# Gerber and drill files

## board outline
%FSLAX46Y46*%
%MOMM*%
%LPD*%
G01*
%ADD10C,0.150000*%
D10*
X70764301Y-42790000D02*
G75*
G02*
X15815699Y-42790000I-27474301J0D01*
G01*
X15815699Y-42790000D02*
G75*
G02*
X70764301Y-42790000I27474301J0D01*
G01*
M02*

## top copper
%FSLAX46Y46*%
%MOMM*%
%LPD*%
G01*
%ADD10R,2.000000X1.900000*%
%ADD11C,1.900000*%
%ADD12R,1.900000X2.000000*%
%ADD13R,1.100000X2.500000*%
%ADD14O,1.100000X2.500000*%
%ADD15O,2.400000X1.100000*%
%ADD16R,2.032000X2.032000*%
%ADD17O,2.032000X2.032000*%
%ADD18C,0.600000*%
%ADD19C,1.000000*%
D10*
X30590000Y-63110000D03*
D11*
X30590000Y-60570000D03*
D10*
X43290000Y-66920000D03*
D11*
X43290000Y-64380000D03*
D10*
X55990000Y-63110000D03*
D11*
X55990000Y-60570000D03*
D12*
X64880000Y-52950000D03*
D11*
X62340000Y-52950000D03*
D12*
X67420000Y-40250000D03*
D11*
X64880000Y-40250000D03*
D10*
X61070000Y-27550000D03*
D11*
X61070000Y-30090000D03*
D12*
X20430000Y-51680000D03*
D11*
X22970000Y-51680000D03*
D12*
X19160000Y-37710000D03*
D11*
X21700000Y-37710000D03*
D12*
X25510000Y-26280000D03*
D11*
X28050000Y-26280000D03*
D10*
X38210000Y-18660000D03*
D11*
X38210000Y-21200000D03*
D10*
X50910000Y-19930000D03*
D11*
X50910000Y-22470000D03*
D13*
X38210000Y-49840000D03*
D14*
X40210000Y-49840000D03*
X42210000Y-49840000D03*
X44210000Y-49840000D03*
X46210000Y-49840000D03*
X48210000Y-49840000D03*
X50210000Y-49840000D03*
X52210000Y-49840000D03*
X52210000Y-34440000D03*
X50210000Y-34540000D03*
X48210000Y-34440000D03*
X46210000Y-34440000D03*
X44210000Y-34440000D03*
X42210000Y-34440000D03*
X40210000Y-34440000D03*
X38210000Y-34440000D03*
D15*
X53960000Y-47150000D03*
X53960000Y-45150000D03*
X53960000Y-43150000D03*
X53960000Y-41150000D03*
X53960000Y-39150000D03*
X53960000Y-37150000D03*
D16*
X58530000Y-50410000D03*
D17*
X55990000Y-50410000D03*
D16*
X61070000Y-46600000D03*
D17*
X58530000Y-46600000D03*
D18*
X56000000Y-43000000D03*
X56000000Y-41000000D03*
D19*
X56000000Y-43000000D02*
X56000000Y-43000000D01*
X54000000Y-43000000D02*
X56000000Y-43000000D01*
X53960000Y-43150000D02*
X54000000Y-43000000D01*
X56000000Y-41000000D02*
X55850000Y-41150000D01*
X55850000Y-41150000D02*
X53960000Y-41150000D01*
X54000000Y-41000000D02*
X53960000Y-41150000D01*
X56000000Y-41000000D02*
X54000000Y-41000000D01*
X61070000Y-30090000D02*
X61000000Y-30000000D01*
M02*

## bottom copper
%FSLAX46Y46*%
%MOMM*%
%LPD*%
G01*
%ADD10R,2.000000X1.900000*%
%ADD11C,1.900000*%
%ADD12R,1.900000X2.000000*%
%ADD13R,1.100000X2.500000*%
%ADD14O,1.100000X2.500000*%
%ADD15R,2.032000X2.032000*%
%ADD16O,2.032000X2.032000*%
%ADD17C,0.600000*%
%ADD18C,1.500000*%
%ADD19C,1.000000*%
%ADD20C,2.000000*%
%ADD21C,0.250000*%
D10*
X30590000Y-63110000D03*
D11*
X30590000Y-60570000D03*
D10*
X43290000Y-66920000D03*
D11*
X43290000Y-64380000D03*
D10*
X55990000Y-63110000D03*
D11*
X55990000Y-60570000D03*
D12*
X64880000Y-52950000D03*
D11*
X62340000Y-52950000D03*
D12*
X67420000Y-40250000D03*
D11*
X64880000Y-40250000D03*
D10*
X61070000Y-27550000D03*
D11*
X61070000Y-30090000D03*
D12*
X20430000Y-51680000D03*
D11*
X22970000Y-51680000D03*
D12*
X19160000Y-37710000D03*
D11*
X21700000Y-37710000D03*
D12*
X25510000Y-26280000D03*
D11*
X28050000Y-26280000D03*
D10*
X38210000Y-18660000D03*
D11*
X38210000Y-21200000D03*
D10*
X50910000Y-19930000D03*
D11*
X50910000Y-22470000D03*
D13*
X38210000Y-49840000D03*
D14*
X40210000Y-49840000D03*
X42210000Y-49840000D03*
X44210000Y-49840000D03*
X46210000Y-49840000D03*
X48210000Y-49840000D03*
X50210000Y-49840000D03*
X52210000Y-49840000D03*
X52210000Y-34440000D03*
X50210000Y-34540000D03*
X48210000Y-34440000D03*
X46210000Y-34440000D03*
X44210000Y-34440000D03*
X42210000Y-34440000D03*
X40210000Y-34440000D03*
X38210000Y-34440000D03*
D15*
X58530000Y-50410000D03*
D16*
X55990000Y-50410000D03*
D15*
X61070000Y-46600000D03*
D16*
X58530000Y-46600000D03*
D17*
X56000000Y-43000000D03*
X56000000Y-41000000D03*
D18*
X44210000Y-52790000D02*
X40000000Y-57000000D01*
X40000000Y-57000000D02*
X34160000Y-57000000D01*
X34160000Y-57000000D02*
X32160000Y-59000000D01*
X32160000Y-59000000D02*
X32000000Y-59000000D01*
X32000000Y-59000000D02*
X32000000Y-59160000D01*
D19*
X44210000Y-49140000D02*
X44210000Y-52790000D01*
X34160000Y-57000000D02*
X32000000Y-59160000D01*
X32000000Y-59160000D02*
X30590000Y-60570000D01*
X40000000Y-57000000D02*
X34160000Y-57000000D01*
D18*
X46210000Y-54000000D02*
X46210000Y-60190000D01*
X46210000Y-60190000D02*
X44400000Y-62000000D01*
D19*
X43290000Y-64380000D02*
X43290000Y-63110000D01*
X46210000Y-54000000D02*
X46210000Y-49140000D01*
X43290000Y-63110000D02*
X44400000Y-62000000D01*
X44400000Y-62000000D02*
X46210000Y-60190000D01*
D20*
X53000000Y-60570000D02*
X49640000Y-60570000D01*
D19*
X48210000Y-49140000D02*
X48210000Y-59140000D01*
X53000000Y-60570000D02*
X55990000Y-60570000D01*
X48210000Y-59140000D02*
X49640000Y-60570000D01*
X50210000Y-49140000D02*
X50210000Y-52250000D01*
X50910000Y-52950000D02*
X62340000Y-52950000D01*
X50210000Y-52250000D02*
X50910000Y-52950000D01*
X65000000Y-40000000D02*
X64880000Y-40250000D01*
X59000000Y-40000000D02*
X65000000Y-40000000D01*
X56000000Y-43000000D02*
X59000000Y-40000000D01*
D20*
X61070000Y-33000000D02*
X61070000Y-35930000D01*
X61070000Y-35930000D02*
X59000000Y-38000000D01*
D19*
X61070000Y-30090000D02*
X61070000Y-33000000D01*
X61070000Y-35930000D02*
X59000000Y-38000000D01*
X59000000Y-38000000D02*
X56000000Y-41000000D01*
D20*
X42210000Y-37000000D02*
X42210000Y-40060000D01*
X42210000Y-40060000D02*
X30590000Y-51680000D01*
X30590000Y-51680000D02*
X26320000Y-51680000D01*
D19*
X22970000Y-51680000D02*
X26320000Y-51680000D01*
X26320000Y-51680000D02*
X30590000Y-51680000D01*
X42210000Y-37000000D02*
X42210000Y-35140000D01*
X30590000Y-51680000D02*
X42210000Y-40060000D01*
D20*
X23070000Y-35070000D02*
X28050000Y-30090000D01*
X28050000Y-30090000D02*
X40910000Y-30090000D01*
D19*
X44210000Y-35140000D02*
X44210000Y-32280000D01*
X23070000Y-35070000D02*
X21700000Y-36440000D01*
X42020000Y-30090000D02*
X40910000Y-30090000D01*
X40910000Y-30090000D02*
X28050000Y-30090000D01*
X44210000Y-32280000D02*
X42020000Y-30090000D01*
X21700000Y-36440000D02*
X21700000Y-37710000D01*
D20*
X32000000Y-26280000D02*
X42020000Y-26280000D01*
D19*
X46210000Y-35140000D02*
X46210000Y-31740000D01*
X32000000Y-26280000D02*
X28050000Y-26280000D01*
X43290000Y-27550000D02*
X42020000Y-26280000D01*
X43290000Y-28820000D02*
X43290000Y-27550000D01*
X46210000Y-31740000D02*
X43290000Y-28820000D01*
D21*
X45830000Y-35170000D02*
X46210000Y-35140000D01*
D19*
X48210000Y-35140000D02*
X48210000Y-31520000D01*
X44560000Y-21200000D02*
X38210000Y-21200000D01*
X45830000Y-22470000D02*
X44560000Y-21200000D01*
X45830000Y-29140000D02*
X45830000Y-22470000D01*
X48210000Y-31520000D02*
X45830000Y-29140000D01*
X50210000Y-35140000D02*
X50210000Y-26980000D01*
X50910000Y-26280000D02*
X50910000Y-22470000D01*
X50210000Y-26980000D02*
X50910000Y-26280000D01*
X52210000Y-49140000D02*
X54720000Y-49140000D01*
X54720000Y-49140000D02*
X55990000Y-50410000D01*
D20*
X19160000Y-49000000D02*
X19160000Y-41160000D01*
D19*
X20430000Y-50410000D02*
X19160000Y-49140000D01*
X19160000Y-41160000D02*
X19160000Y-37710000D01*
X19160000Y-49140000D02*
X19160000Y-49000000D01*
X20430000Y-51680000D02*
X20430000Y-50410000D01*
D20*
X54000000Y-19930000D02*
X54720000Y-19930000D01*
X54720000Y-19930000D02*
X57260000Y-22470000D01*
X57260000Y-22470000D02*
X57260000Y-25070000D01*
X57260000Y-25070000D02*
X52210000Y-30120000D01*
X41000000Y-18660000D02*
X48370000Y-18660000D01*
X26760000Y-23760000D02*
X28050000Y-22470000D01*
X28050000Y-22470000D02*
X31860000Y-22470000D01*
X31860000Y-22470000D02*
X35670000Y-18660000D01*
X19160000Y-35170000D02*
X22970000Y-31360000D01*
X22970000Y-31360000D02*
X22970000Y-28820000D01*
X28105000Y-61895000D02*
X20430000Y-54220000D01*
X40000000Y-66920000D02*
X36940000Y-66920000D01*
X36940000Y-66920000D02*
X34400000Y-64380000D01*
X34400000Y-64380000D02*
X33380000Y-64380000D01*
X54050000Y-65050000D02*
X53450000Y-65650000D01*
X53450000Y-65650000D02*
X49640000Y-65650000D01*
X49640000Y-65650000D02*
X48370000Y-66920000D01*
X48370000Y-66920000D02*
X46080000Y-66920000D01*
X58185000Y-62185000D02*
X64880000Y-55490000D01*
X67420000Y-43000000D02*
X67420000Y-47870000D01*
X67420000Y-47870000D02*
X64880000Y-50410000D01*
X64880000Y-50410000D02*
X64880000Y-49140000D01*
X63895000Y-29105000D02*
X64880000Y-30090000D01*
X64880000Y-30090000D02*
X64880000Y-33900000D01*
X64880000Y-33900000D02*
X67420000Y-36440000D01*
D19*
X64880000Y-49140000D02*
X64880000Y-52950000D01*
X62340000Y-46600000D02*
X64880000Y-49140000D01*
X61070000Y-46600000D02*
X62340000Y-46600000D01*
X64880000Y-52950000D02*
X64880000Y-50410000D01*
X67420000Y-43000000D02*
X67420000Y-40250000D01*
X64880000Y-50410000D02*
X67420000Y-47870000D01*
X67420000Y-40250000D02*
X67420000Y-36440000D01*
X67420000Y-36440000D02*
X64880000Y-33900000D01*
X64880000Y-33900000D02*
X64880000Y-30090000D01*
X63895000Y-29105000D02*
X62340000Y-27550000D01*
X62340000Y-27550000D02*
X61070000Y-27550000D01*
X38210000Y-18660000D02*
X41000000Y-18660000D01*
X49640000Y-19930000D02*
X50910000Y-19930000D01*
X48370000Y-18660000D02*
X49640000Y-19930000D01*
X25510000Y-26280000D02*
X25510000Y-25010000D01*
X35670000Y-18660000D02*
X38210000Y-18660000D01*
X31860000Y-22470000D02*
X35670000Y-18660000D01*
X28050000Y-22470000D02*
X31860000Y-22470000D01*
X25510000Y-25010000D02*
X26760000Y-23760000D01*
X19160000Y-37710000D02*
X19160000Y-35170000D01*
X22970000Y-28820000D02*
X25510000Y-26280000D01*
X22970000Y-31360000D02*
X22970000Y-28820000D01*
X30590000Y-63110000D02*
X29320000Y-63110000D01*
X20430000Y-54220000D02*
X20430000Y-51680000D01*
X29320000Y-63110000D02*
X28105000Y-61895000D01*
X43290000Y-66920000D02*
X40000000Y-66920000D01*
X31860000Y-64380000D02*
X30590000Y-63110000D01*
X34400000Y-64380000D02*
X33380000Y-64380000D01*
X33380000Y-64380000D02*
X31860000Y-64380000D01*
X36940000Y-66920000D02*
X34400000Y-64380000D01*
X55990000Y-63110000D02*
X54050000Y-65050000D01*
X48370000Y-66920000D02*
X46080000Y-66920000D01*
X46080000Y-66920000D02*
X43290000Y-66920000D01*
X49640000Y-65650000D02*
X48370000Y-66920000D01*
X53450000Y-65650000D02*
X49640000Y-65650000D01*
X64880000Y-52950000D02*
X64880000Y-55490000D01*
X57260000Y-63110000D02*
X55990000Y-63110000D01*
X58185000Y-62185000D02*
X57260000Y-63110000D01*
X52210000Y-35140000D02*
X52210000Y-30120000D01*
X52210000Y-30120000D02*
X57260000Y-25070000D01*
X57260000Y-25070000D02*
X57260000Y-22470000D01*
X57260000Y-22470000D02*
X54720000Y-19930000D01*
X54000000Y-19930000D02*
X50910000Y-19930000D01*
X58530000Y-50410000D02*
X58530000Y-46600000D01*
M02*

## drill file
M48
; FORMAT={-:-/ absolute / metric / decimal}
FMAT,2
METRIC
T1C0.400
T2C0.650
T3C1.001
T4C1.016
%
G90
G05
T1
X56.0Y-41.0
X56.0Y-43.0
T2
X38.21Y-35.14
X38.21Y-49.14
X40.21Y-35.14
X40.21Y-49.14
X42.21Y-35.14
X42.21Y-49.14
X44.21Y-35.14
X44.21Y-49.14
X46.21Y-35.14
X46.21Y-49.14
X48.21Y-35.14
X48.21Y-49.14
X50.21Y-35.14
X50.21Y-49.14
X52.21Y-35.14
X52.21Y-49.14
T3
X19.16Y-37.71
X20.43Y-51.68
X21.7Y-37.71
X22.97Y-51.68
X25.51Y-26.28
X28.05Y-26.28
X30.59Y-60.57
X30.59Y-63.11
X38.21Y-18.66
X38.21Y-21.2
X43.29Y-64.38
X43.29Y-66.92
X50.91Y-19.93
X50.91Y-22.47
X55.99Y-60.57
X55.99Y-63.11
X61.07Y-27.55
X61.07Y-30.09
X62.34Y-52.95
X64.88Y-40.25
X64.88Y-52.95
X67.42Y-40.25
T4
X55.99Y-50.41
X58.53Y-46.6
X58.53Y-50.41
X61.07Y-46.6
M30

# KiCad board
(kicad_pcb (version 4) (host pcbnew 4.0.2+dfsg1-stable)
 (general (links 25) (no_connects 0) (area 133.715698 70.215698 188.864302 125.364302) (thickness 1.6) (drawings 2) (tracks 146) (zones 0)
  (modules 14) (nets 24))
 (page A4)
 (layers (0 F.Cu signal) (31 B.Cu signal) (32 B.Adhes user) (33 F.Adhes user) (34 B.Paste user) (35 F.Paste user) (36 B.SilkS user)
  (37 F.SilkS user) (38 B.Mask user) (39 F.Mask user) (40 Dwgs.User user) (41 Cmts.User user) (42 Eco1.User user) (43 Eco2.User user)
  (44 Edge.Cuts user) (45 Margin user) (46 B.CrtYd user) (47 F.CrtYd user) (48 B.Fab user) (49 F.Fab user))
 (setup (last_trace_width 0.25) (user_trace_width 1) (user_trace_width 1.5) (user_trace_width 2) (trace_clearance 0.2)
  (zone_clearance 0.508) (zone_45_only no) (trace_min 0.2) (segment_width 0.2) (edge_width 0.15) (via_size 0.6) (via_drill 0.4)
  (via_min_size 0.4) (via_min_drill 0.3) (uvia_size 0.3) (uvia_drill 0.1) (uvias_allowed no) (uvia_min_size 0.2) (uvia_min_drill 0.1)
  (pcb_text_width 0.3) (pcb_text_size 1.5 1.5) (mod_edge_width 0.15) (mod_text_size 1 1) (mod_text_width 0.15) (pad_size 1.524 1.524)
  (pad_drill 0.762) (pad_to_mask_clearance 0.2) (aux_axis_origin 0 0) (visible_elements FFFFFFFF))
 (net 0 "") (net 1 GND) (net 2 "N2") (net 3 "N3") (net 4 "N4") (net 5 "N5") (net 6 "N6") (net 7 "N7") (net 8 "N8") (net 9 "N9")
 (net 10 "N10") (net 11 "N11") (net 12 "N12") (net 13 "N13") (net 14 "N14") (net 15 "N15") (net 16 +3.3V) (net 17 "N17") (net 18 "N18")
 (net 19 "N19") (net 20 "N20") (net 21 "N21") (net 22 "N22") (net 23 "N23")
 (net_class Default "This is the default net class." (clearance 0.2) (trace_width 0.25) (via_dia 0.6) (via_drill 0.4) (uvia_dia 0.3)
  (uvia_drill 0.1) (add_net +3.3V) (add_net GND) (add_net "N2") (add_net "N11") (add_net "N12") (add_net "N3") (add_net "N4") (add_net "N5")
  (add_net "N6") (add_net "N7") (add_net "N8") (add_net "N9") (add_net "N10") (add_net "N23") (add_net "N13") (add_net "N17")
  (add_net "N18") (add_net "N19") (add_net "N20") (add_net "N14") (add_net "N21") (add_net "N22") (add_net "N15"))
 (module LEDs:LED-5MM (layer F.Cu) (at 30.59 63.11 90)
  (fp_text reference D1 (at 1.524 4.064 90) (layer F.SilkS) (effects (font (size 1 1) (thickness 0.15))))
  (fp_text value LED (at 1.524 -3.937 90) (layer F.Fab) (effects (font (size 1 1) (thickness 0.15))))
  (pad 1 thru_hole rect (at 0 0 180) (size 2 1.9) (drill 1.00076) (layers *.Cu *.Mask F.SilkS) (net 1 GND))
  (pad 2 thru_hole circle (at 2.54 0 90) (size 1.9 1.9) (drill 1.00076) (layers *.Cu *.Mask F.SilkS) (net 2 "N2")))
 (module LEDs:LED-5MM (layer F.Cu) (at 43.29 66.92 90)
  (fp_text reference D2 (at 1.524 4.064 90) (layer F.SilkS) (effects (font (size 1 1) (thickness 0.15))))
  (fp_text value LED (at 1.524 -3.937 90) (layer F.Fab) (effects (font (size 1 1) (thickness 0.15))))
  (pad 1 thru_hole rect (at 0 0 180) (size 2 1.9) (drill 1.00076) (layers *.Cu *.Mask F.SilkS) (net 1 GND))
  (pad 2 thru_hole circle (at 2.54 0 90) (size 1.9 1.9) (drill 1.00076) (layers *.Cu *.Mask F.SilkS) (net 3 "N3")))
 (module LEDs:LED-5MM (layer F.Cu) (at 55.99 63.11 90)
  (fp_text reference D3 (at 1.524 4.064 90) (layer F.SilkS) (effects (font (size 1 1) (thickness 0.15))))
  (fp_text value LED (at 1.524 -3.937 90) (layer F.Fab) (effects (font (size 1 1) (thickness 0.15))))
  (pad 1 thru_hole rect (at 0 0 180) (size 2 1.9) (drill 1.00076) (layers *.Cu *.Mask F.SilkS) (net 1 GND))
  (pad 2 thru_hole circle (at 2.54 0 90) (size 1.9 1.9) (drill 1.00076) (layers *.Cu *.Mask F.SilkS) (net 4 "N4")))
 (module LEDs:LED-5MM (layer F.Cu) (at 64.88 52.95 180)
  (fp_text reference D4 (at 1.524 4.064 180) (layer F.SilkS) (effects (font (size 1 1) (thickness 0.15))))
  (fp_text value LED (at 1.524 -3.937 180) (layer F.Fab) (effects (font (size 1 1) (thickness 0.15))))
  (pad 1 thru_hole rect (at 0 0 270) (size 2 1.9) (drill 1.00076) (layers *.Cu *.Mask F.SilkS) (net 1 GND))
  (pad 2 thru_hole circle (at 2.54 0 180) (size 1.9 1.9) (drill 1.00076) (layers *.Cu *.Mask F.SilkS) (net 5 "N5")))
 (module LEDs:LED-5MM (layer F.Cu) (at 67.42 40.25 180)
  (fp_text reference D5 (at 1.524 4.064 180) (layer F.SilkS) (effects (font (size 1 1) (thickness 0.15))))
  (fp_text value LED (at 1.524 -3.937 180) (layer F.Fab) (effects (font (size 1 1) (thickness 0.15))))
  (pad 1 thru_hole rect (at 0 0 270) (size 2 1.9) (drill 1.00076) (layers *.Cu *.Mask F.SilkS) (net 1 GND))
  (pad 2 thru_hole circle (at 2.54 0 180) (size 1.9 1.9) (drill 1.00076) (layers *.Cu *.Mask F.SilkS) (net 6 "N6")))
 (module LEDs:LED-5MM (layer F.Cu) (at 61.07 27.55 270)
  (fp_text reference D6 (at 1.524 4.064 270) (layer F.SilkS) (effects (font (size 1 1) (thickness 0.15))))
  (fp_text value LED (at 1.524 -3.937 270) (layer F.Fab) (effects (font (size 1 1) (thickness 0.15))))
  (pad 1 thru_hole rect (at 0 0) (size 2 1.9) (drill 1.00076) (layers *.Cu *.Mask F.SilkS) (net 1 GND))
  (pad 2 thru_hole circle (at 2.54 0 270) (size 1.9 1.9) (drill 1.00076) (layers *.Cu *.Mask F.SilkS) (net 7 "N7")))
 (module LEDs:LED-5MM (layer F.Cu) (at 20.43 51.68)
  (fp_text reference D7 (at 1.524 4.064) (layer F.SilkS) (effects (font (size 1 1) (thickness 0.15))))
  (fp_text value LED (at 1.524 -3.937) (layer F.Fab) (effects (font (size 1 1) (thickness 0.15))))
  (pad 1 thru_hole rect (at 0 0 90) (size 2 1.9) (drill 1.00076) (layers *.Cu *.Mask F.SilkS) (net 1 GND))
  (pad 2 thru_hole circle (at 2.54 0) (size 1.9 1.9) (drill 1.00076) (layers *.Cu *.Mask F.SilkS) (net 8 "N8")))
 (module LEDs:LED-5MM (layer F.Cu) (at 19.16 37.71)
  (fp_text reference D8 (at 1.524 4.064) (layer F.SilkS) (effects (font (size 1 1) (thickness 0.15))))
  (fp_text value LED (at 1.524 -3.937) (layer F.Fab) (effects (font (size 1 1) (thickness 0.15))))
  (pad 1 thru_hole rect (at 0 0 90) (size 2 1.9) (drill 1.00076) (layers *.Cu *.Mask F.SilkS) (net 1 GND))
  (pad 2 thru_hole circle (at 2.54 0) (size 1.9 1.9) (drill 1.00076) (layers *.Cu *.Mask F.SilkS) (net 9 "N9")))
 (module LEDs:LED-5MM (layer F.Cu) (at 25.51 26.28)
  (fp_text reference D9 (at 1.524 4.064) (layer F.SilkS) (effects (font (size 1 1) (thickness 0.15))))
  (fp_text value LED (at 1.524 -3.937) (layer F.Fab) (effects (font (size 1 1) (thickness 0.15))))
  (pad 1 thru_hole rect (at 0 0 90) (size 2 1.9) (drill 1.00076) (layers *.Cu *.Mask F.SilkS) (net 1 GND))
  (pad 2 thru_hole circle (at 2.54 0) (size 1.9 1.9) (drill 1.00076) (layers *.Cu *.Mask F.SilkS) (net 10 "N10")))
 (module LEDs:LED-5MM (layer F.Cu) (at 38.21 18.66 270)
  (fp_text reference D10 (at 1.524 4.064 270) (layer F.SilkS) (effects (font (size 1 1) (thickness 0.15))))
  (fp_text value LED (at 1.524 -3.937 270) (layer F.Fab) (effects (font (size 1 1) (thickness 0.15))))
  (pad 1 thru_hole rect (at 0 0) (size 2 1.9) (drill 1.00076) (layers *.Cu *.Mask F.SilkS) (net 1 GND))
  (pad 2 thru_hole circle (at 2.54 0 270) (size 1.9 1.9) (drill 1.00076) (layers *.Cu *.Mask F.SilkS) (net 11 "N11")))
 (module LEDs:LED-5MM (layer F.Cu) (at 50.91 19.93 270)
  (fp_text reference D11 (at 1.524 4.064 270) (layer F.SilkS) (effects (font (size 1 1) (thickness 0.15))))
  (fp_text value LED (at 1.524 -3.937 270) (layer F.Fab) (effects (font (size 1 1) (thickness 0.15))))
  (pad 1 thru_hole rect (at 0 0) (size 2 1.9) (drill 1.00076) (layers *.Cu *.Mask F.SilkS) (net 1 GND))
  (pad 2 thru_hole circle (at 2.54 0 270) (size 1.9 1.9) (drill 1.00076) (layers *.Cu *.Mask F.SilkS) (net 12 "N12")))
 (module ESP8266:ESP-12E (layer F.Cu) (at 38.21 49.14 90)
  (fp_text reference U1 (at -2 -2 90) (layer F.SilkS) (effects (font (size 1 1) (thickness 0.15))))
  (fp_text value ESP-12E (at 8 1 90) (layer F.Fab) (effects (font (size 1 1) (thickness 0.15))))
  (pad 1 thru_hole rect (at 0 0 90) (size 2.5 1.1) (drill 0.65 (offset -0.7 0)) (layers *.Cu *.Mask F.SilkS) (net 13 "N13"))
  (pad 2 thru_hole oval (at 0 2 90) (size 2.5 1.1) (drill 0.65 (offset -0.7 0)) (layers *.Cu *.Mask F.SilkS) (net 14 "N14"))
  (pad 3 thru_hole oval (at 0 4 90) (size 2.5 1.1) (drill 0.65 (offset -0.7 0)) (layers *.Cu *.Mask F.SilkS) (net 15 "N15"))
  (pad 4 thru_hole oval (at 0 6 90) (size 2.5 1.1) (drill 0.65 (offset -0.7 0)) (layers *.Cu *.Mask F.SilkS) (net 2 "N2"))
  (pad 5 thru_hole oval (at 0 8 90) (size 2.5 1.1) (drill 0.65 (offset -0.7 0)) (layers *.Cu *.Mask F.SilkS) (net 3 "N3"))
  (pad 6 thru_hole oval (at 0 10 90) (size 2.5 1.1) (drill 0.65 (offset -0.7 0)) (layers *.Cu *.Mask F.SilkS) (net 4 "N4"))
  (pad 7 thru_hole oval (at 0 12 90) (size 2.5 1.1) (drill 0.65 (offset -0.7 0)) (layers *.Cu *.Mask F.SilkS) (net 5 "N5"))
  (pad 8 thru_hole oval (at 0 14 90) (size 2.5 1.1) (drill 0.65 (offset -0.7 0)) (layers *.Cu *.Mask F.SilkS) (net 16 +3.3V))
  (pad 9 thru_hole oval (at 14 14 90) (size 2.5 1.1) (drill 0.65 (offset 0.7 0)) (layers *.Cu *.Mask F.SilkS) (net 1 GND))
  (pad 10 thru_hole oval (at 14 12 90) (size 2.5 1.1) (drill 0.65 (offset 0.6 0)) (layers *.Cu *.Mask F.SilkS) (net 12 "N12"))
  (pad 11 thru_hole oval (at 14 10 90) (size 2.5 1.1) (drill 0.65 (offset 0.7 0)) (layers *.Cu *.Mask F.SilkS) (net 11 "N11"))
  (pad 12 thru_hole oval (at 14 8 90) (size 2.5 1.1) (drill 0.65 (offset 0.7 0)) (layers *.Cu *.Mask F.SilkS) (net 10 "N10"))
  (pad 13 thru_hole oval (at 14 6 90) (size 2.5 1.1) (drill 0.65 (offset 0.7 0)) (layers *.Cu *.Mask F.SilkS) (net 9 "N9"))
  (pad 14 thru_hole oval (at 14 4 90) (size 2.5 1.1) (drill 0.65 (offset 0.7 0)) (layers *.Cu *.Mask F.SilkS) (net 8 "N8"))
  (pad 15 thru_hole oval (at 14 2 90) (size 2.5 1.1) (drill 0.65 (offset 0.7 0)) (layers *.Cu *.Mask F.SilkS) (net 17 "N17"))
  (pad 16 thru_hole oval (at 14 0 90) (size 2.5 1.1) (drill 0.65 (offset 0.7 0)) (layers *.Cu *.Mask F.SilkS) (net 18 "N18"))
  (pad 17 smd oval (at 1.99 15.75 180) (size 2.4 1.1) (layers F.Cu F.Paste F.Mask) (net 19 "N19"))
  (pad 18 smd oval (at 3.99 15.75 180) (size 2.4 1.1) (layers F.Cu F.Paste F.Mask) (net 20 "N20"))
  (pad 19 smd oval (at 5.99 15.75 180) (size 2.4 1.1) (layers F.Cu F.Paste F.Mask) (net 6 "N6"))
  (pad 20 smd oval (at 7.99 15.75 180) (size 2.4 1.1) (layers F.Cu F.Paste F.Mask) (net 7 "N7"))
  (pad 21 smd oval (at 9.99 15.75 180) (size 2.4 1.1) (layers F.Cu F.Paste F.Mask) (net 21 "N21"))
  (pad 22 smd oval (at 11.99 15.75 180) (size 2.4 1.1) (layers F.Cu F.Paste F.Mask) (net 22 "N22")))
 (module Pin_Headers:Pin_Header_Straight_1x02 (layer F.Cu) (at 58.53 50.41 270)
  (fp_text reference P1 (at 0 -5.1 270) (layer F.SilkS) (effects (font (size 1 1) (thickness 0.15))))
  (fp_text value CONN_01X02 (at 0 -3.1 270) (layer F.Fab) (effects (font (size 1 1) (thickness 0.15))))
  (pad 1 thru_hole rect (at 0 0 270) (size 2.032 2.032) (drill 1.016) (layers *.Cu *.Mask F.SilkS) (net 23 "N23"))
  (pad 2 thru_hole oval (at 0 2.54 270) (size 2.032 2.032) (drill 1.016) (layers *.Cu *.Mask F.SilkS) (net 16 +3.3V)))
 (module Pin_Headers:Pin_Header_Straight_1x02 (layer F.Cu) (at 61.07 46.6 270)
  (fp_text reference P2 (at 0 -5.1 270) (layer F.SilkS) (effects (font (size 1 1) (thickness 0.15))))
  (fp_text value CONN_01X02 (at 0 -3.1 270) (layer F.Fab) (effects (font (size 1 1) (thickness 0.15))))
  (pad 1 thru_hole rect (at 0 0 270) (size 2.032 2.032) (drill 1.016) (layers *.Cu *.Mask F.SilkS) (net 1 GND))
  (pad 2 thru_hole oval (at 0 2.54 270) (size 2.032 2.032) (drill 1.016) (layers *.Cu *.Mask F.SilkS) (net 23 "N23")))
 (gr_circle (center 43.29 42.79) (end 66.15 58.03) (layer Edge.Cuts) (width 0.15))
 (segment (start 44.21 52.79) (end 40 57) (width 1.5) (layer B.Cu) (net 2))
 (segment (start 40 57) (end 34.16 57) (width 1.5) (layer B.Cu) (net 2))
 (segment (start 34.16 57) (end 32.16 59) (width 1.5) (layer B.Cu) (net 2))
 (segment (start 32.16 59) (end 32 59) (width 1.5) (layer B.Cu) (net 2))
 (segment (start 32 59) (end 32 59.16) (width 1.5) (layer B.Cu) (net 2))
 (segment (start 44.21 49.14) (end 44.21 52.79) (width 1) (layer B.Cu) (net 2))
 (segment (start 34.16 57) (end 32 59.16) (width 1) (layer B.Cu) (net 2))
 (segment (start 32 59.16) (end 30.59 60.57) (width 1) (layer B.Cu) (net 2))
 (segment (start 40 57) (end 34.16 57) (width 1) (layer B.Cu) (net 2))
 (segment (start 46.21 54) (end 46.21 60.19) (width 1.5) (layer B.Cu) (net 3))
 (segment (start 46.21 60.19) (end 44.4 62) (width 1.5) (layer B.Cu) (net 3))
 (segment (start 43.29 64.38) (end 43.29 63.11) (width 1) (layer B.Cu) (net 3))
 (segment (start 46.21 54) (end 46.21 49.14) (width 1) (layer B.Cu) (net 3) (status 20))
 (segment (start 43.29 63.11) (end 44.4 62) (width 1) (layer B.Cu) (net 3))
 (segment (start 44.4 62) (end 46.21 60.19) (width 1) (layer B.Cu) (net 3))
 (segment (start 53 60.57) (end 49.64 60.57) (width 2) (layer B.Cu) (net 4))
 (segment (start 48.21 49.14) (end 48.21 59.14) (width 1) (layer B.Cu) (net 4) (status 10))
 (segment (start 53 60.57) (end 55.99 60.57) (width 1) (layer B.Cu) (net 4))
 (segment (start 48.21 59.14) (end 49.64 60.57) (width 1) (layer B.Cu) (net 4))
 (segment (start 50.21 49.14) (end 50.21 52.25) (width 1) (layer B.Cu) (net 5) (status 10))
 (segment (start 50.91 52.95) (end 62.34 52.95) (width 1) (layer B.Cu) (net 5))
 (segment (start 50.21 52.25) (end 50.91 52.95) (width 1) (layer B.Cu) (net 5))
 (segment (start 65 40) (end 64.88 40.25) (width 1) (layer B.Cu) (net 6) (status 80000))
 (segment (start 59 40) (end 65 40) (width 1) (layer B.Cu) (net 6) (status 80000))
 (segment (start 56 43) (end 59 40) (width 1) (layer B.Cu) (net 6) (status 80000))
 (via (at 56 43) (size 0.6) (layers F.Cu B.Cu) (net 6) (status 80000))
 (segment (start 56 43) (end 56 43) (width 1) (layer F.Cu) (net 6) (status 80000))
 (segment (start 54 43) (end 56 43) (width 1) (layer F.Cu) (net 6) (status 80000))
 (segment (start 53.96 43.15) (end 54 43) (width 1) (layer F.Cu) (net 6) (status 80000))
 (segment (start 61.07 33) (end 61.07 35.93) (width 2) (layer B.Cu) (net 7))
 (segment (start 61.07 35.93) (end 59 38) (width 2) (layer B.Cu) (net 7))
 (segment (start 61.07 30.09) (end 61.07 33) (width 1) (layer B.Cu) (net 7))
 (via (at 56 41) (size 0.6) (drill 0.4) (layers F.Cu B.Cu) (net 7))
 (segment (start 61.07 35.93) (end 59 38) (width 1) (layer B.Cu) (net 7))
 (segment (start 59 38) (end 56 41) (width 1) (layer B.Cu) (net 7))
 (segment (start 56 41) (end 55.85 41.15) (width 1) (layer F.Cu) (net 7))
 (segment (start 55.85 41.15) (end 53.96 41.15) (width 1) (layer F.Cu) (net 7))
 (segment (start 54 41) (end 53.96 41.15) (width 1) (layer F.Cu) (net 7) (status 80000))
 (segment (start 56 41) (end 54 41) (width 1) (layer F.Cu) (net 7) (status 80000))
 (segment (start 61.07 30.09) (end 61 30) (width 1) (layer F.Cu) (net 7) (status 80000))
 (segment (start 42.21 37) (end 42.21 40.06) (width 2) (layer B.Cu) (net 8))
 (segment (start 42.21 40.06) (end 30.59 51.68) (width 2) (layer B.Cu) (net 8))
 (segment (start 30.59 51.68) (end 26.32 51.68) (width 2) (layer B.Cu) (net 8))
 (segment (start 22.97 51.68) (end 26.32 51.68) (width 1) (layer B.Cu) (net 8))
 (segment (start 26.32 51.68) (end 30.59 51.68) (width 1) (layer B.Cu) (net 8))
 (segment (start 42.21 37) (end 42.21 35.14) (width 1) (layer B.Cu) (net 8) (status 20))
 (segment (start 30.59 51.68) (end 42.21 40.06) (width 1) (layer B.Cu) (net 8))
 (segment (start 23.07 35.07) (end 28.05 30.09) (width 2) (layer B.Cu) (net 9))
 (segment (start 28.05 30.09) (end 40.91 30.09) (width 2) (layer B.Cu) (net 9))
 (segment (start 44.21 35.14) (end 44.21 32.28) (width 1) (layer B.Cu) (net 9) (status 10))
 (segment (start 23.07 35.07) (end 21.7 36.44) (width 1) (layer B.Cu) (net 9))
 (segment (start 42.02 30.09) (end 40.91 30.09) (width 1) (layer B.Cu) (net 9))
 (segment (start 40.91 30.09) (end 28.05 30.09) (width 1) (layer B.Cu) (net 9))
 (segment (start 44.21 32.28) (end 42.02 30.09) (width 1) (layer B.Cu) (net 9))
 (segment (start 21.7 36.44) (end 21.7 37.71) (width 1) (layer B.Cu) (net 9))
 (segment (start 32 26.28) (end 42.02 26.28) (width 2) (layer B.Cu) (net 10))
 (segment (start 46.21 35.14) (end 46.21 31.74) (width 1) (layer B.Cu) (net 10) (status 10))
 (segment (start 32 26.28) (end 28.05 26.28) (width 1) (layer B.Cu) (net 10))
 (segment (start 43.29 27.55) (end 42.02 26.28) (width 1) (layer B.Cu) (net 10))
 (segment (start 43.29 28.82) (end 43.29 27.55) (width 1) (layer B.Cu) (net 10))
 (segment (start 46.21 31.74) (end 43.29 28.82) (width 1) (layer B.Cu) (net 10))
 (segment (start 45.83 35.17) (end 46.21 35.14) (width 0.25) (layer B.Cu) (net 10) (status 80030))
 (segment (start 48.21 35.14) (end 48.21 31.52) (width 1) (layer B.Cu) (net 11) (status 10))
 (segment (start 44.56 21.2) (end 38.21 21.2) (width 1) (layer B.Cu) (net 11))
 (segment (start 45.83 22.47) (end 44.56 21.2) (width 1) (layer B.Cu) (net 11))
 (segment (start 45.83 29.14) (end 45.83 22.47) (width 1) (layer B.Cu) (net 11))
 (segment (start 48.21 31.52) (end 45.83 29.14) (width 1) (layer B.Cu) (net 11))
 (segment (start 50.21 35.14) (end 50.21 26.98) (width 1) (layer B.Cu) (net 12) (status 10))
 (segment (start 50.91 26.28) (end 50.91 22.47) (width 1) (layer B.Cu) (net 12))
 (segment (start 50.21 26.98) (end 50.91 26.28) (width 1) (layer B.Cu) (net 12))
 (segment (start 52.21 49.14) (end 54.72 49.14) (width 1) (layer B.Cu) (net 16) (status 10))
 (segment (start 54.72 49.14) (end 55.99 50.41) (width 1) (layer B.Cu) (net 16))
 (segment (start 19.16 49) (end 19.16 41.16) (width 2) (layer B.Cu) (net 1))
 (segment (start 20.43 50.41) (end 19.16 49.14) (width 1) (layer B.Cu) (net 1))
 (segment (start 19.16 41.16) (end 19.16 37.71) (width 1) (layer B.Cu) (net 1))
 (segment (start 19.16 49.14) (end 19.16 49) (width 1) (layer B.Cu) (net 1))
 (segment (start 20.43 51.68) (end 20.43 50.41) (width 1) (layer B.Cu) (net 1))
 (segment (start 54 19.93) (end 54.72 19.93) (width 2) (layer B.Cu) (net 1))
 (segment (start 54.72 19.93) (end 57.26 22.47) (width 2) (layer B.Cu) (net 1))
 (segment (start 57.26 22.47) (end 57.26 25.07) (width 2) (layer B.Cu) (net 1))
 (segment (start 57.26 25.07) (end 52.21 30.12) (width 2) (layer B.Cu) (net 1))
 (segment (start 41 18.66) (end 48.37 18.66) (width 2) (layer B.Cu) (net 1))
 (segment (start 26.76 23.76) (end 28.05 22.47) (width 2) (layer B.Cu) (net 1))
 (segment (start 28.05 22.47) (end 31.86 22.47) (width 2) (layer B.Cu) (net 1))
 (segment (start 31.86 22.47) (end 35.67 18.66) (width 2) (layer B.Cu) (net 1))
 (segment (start 19.16 35.17) (end 22.97 31.36) (width 2) (layer B.Cu) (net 1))
 (segment (start 22.97 31.36) (end 22.97 28.82) (width 2) (layer B.Cu) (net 1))
 (segment (start 28.105 61.895) (end 20.43 54.22) (width 2) (layer B.Cu) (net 1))
 (segment (start 40 66.92) (end 36.94 66.92) (width 2) (layer B.Cu) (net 1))
 (segment (start 36.94 66.92) (end 34.4 64.38) (width 2) (layer B.Cu) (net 1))
 (segment (start 34.4 64.38) (end 33.38 64.38) (width 2) (layer B.Cu) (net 1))
 (segment (start 54.05 65.05) (end 53.45 65.65) (width 2) (layer B.Cu) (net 1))
 (segment (start 53.45 65.65) (end 49.64 65.65) (width 2) (layer B.Cu) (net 1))
 (segment (start 49.64 65.65) (end 48.37 66.92) (width 2) (layer B.Cu) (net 1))
 (segment (start 48.37 66.92) (end 46.08 66.92) (width 2) (layer B.Cu) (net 1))
 (segment (start 58.185 62.185) (end 64.88 55.49) (width 2) (layer B.Cu) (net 1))
 (segment (start 67.42 43) (end 67.42 47.87) (width 2) (layer B.Cu) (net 1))
 (segment (start 67.42 47.87) (end 64.88 50.41) (width 2) (layer B.Cu) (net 1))
 (segment (start 64.88 50.41) (end 64.88 49.14) (width 2) (layer B.Cu) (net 1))
 (segment (start 63.895 29.105) (end 64.88 30.09) (width 2) (layer B.Cu) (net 1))
 (segment (start 64.88 30.09) (end 64.88 33.9) (width 2) (layer B.Cu) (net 1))
 (segment (start 64.88 33.9) (end 67.42 36.44) (width 2) (layer B.Cu) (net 1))
 (segment (start 64.88 49.14) (end 64.88 52.95) (width 1) (layer B.Cu) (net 1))
 (segment (start 62.34 46.6) (end 64.88 49.14) (width 1) (layer B.Cu) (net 1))
 (segment (start 61.07 46.6) (end 62.34 46.6) (width 1) (layer B.Cu) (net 1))
 (segment (start 64.88 52.95) (end 64.88 50.41) (width 1) (layer B.Cu) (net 1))
 (segment (start 67.42 43) (end 67.42 40.25) (width 1) (layer B.Cu) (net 1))
 (segment (start 64.88 50.41) (end 67.42 47.87) (width 1) (layer B.Cu) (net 1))
 (segment (start 67.42 40.25) (end 67.42 36.44) (width 1) (layer B.Cu) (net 1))
 (segment (start 67.42 36.44) (end 64.88 33.9) (width 1) (layer B.Cu) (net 1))
 (segment (start 64.88 33.9) (end 64.88 30.09) (width 1) (layer B.Cu) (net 1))
 (segment (start 63.895 29.105) (end 62.34 27.55) (width 1) (layer B.Cu) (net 1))
 (segment (start 62.34 27.55) (end 61.07 27.55) (width 1) (layer B.Cu) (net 1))
 (segment (start 38.21 18.66) (end 41 18.66) (width 1) (layer B.Cu) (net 1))
 (segment (start 49.64 19.93) (end 50.91 19.93) (width 1) (layer B.Cu) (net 1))
 (segment (start 48.37 18.66) (end 49.64 19.93) (width 1) (layer B.Cu) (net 1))
 (segment (start 25.51 26.28) (end 25.51 25.01) (width 1) (layer B.Cu) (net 1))
 (segment (start 35.67 18.66) (end 38.21 18.66) (width 1) (layer B.Cu) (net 1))
 (segment (start 31.86 22.47) (end 35.67 18.66) (width 1) (layer B.Cu) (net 1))
 (segment (start 28.05 22.47) (end 31.86 22.47) (width 1) (layer B.Cu) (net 1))
 (segment (start 25.51 25.01) (end 26.76 23.76) (width 1) (layer B.Cu) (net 1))
 (segment (start 19.16 37.71) (end 19.16 35.17) (width 1) (layer B.Cu) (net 1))
 (segment (start 22.97 28.82) (end 25.51 26.28) (width 1) (layer B.Cu) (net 1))
 (segment (start 22.97 31.36) (end 22.97 28.82) (width 1) (layer B.Cu) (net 1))
 (segment (start 30.59 63.11) (end 29.32 63.11) (width 1) (layer B.Cu) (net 1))
 (segment (start 20.43 54.22) (end 20.43 51.68) (width 1) (layer B.Cu) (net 1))
 (segment (start 29.32 63.11) (end 28.105 61.895) (width 1) (layer B.Cu) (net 1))
 (segment (start 43.29 66.92) (end 40 66.92) (width 1) (layer B.Cu) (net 1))
 (segment (start 31.86 64.38) (end 30.59 63.11) (width 1) (layer B.Cu) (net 1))
 (segment (start 34.4 64.38) (end 33.38 64.38) (width 1) (layer B.Cu) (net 1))
 (segment (start 33.38 64.38) (end 31.86 64.38) (width 1) (layer B.Cu) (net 1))
 (segment (start 36.94 66.92) (end 34.4 64.38) (width 1) (layer B.Cu) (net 1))
 (segment (start 55.99 63.11) (end 54.05 65.05) (width 1) (layer B.Cu) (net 1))
 (segment (start 48.37 66.92) (end 46.08 66.92) (width 1) (layer B.Cu) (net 1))
 (segment (start 46.08 66.92) (end 43.29 66.92) (width 1) (layer B.Cu) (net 1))
 (segment (start 49.64 65.65) (end 48.37 66.92) (width 1) (layer B.Cu) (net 1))
 (segment (start 53.45 65.65) (end 49.64 65.65) (width 1) (layer B.Cu) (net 1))
 (segment (start 64.88 52.95) (end 64.88 55.49) (width 1) (layer B.Cu) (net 1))
 (segment (start 57.26 63.11) (end 55.99 63.11) (width 1) (layer B.Cu) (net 1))
 (segment (start 58.185 62.185) (end 57.26 63.11) (width 1) (layer B.Cu) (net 1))
 (segment (start 52.21 35.14) (end 52.21 30.12) (width 1) (layer B.Cu) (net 1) (status 10))
 (segment (start 52.21 30.12) (end 57.26 25.07) (width 1) (layer B.Cu) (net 1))
 (segment (start 57.26 25.07) (end 57.26 22.47) (width 1) (layer B.Cu) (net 1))
 (segment (start 57.26 22.47) (end 54.72 19.93) (width 1) (layer B.Cu) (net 1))
 (segment (start 54 19.93) (end 50.91 19.93) (width 1) (layer B.Cu) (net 1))
 (segment (start 58.53 50.41) (end 58.53 46.6) (width 1) (layer B.Cu) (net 23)))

